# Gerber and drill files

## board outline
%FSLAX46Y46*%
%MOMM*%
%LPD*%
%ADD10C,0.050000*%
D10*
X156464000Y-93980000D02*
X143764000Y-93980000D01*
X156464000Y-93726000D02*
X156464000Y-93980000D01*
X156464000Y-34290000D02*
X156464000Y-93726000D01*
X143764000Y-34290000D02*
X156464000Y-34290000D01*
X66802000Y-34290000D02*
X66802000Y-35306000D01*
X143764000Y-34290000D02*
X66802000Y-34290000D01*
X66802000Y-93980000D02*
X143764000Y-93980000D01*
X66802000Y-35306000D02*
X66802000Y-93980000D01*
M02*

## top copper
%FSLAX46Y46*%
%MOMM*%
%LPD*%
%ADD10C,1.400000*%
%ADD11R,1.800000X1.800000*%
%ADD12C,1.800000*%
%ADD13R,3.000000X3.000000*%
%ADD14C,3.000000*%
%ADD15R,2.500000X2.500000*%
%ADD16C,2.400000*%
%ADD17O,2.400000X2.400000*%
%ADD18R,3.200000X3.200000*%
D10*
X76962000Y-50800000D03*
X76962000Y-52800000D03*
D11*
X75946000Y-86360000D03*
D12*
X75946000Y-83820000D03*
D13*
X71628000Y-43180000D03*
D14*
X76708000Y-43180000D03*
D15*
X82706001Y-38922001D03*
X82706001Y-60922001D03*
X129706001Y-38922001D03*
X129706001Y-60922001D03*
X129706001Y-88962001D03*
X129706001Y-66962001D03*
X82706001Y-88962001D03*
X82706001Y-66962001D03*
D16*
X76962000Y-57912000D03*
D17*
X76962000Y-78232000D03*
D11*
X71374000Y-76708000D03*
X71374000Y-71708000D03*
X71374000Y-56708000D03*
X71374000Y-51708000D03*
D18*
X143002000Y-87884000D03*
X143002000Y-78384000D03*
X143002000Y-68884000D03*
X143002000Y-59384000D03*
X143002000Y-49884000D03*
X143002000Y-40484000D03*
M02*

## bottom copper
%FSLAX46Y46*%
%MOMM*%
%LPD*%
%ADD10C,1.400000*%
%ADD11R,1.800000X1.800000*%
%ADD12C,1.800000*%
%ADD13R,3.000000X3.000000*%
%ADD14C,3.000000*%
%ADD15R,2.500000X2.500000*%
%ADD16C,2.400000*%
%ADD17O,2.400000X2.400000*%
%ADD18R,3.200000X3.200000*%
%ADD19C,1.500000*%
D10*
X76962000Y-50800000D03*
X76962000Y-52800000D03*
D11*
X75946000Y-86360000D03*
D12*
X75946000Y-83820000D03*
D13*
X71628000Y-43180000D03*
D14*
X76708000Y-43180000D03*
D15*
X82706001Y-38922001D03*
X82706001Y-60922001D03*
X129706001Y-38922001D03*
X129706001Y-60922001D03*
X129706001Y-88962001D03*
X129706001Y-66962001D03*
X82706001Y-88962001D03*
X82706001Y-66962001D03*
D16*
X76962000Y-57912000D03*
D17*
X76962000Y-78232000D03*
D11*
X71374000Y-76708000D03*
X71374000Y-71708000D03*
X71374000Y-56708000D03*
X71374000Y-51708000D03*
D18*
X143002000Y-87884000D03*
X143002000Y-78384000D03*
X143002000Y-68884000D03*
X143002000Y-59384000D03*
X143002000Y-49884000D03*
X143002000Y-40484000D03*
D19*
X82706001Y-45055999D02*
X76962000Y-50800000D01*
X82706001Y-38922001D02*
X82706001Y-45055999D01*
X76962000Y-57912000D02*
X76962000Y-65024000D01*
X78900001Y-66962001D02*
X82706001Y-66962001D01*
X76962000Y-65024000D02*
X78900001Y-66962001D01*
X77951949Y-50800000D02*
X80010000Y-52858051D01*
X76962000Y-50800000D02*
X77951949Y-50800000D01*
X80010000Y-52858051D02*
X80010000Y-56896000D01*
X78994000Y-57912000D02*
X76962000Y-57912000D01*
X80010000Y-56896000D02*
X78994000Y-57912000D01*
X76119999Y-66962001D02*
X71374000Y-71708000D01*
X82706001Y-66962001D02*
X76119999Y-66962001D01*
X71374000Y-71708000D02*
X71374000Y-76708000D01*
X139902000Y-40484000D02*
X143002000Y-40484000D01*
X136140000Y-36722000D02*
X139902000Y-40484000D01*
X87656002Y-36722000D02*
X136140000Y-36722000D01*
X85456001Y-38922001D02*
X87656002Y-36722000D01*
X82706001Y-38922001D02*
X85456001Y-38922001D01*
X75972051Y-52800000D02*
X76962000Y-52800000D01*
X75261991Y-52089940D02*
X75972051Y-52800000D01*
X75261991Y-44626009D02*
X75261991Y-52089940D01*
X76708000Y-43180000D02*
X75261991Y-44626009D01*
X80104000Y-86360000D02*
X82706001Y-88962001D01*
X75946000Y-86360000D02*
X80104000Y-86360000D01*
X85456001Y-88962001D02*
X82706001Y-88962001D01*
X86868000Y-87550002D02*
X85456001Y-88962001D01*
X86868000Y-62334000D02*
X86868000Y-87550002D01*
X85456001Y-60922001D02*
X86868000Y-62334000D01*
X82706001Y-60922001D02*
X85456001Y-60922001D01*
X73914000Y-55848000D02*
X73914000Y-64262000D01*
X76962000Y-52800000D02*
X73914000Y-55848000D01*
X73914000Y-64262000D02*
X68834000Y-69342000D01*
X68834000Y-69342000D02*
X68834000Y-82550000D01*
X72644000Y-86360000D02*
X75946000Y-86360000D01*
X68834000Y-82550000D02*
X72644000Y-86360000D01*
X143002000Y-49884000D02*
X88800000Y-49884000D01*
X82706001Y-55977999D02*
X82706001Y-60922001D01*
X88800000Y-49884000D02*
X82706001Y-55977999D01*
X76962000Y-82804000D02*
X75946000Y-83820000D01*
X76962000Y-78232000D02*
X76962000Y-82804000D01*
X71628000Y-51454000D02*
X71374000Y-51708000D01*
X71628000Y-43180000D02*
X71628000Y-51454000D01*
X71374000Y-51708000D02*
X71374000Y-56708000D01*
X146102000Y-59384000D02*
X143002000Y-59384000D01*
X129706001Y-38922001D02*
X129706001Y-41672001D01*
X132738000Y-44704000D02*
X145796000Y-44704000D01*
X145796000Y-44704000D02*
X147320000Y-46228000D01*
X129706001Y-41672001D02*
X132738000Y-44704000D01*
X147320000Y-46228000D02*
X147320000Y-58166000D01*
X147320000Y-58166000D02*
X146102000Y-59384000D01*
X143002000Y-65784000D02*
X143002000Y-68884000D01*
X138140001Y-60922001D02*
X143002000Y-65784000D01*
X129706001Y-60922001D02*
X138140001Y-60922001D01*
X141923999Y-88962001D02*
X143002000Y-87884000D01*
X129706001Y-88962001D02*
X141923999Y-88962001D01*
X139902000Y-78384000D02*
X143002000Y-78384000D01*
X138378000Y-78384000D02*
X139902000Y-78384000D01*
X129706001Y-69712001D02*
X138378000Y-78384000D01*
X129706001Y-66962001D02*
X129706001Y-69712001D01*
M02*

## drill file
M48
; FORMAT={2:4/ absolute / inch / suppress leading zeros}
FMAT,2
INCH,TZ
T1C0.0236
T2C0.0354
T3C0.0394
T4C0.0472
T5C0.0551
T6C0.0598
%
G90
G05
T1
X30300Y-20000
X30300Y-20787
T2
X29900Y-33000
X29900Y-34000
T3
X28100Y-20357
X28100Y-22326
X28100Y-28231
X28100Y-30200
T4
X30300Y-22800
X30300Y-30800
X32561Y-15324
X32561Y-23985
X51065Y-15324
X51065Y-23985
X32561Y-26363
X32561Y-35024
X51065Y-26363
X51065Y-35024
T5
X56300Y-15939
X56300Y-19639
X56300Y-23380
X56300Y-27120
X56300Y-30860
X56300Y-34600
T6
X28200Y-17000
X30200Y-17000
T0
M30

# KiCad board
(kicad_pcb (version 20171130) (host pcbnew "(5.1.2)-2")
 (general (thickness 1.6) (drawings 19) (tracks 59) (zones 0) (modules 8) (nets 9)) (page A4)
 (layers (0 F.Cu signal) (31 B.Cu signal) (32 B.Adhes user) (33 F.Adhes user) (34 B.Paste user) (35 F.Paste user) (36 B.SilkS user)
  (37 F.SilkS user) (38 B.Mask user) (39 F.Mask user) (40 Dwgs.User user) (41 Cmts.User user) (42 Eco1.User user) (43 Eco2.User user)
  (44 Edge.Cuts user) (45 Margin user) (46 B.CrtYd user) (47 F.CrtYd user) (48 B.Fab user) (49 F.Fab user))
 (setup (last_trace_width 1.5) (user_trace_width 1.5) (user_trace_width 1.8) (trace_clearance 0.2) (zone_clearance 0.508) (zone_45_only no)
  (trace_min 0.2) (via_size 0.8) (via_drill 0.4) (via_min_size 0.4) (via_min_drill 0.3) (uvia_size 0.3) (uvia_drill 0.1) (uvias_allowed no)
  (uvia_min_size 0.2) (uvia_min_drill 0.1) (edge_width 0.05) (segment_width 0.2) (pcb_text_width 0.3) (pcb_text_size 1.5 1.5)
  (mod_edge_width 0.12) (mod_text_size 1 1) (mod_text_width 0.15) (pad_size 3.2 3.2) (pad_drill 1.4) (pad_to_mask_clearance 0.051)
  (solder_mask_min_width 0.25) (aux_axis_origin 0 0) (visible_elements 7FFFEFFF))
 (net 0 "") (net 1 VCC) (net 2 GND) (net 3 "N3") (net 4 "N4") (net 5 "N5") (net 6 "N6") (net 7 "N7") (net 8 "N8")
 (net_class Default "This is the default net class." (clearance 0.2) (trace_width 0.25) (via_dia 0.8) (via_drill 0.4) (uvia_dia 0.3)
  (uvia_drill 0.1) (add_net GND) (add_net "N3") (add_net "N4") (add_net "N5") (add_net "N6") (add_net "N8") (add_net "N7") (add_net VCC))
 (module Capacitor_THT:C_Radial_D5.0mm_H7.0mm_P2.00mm (layer F.Cu) (at 76.962 50.8 270)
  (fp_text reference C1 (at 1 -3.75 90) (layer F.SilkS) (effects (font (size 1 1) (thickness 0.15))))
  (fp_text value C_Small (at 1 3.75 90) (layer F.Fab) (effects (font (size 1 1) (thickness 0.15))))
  (pad 1 thru_hole circle (at 0 0 270) (size 1.4 1.4) (drill 0.6) (layers *.Cu *.Mask) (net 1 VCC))
  (pad 2 thru_hole circle (at 2 0 270) (size 1.4 1.4) (drill 0.6) (layers *.Cu *.Mask) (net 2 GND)))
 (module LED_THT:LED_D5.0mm (layer F.Cu) (at 75.946 86.36 90)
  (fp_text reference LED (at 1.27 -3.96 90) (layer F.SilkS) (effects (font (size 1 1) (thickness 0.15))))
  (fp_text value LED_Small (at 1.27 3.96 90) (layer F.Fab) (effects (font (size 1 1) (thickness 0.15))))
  (pad 1 thru_hole rect (at 0 0 90) (size 1.8 1.8) (drill 0.9) (layers *.Cu *.Mask) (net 2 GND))
  (pad 2 thru_hole circle (at 2.54 0 90) (size 1.8 1.8) (drill 0.9) (layers *.Cu *.Mask) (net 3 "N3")))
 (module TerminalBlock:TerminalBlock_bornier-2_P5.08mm (layer F.Cu) (at 71.628 43.18)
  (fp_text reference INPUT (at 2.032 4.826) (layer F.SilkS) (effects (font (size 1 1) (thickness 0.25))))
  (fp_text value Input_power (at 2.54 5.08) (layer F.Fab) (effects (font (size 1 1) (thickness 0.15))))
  (pad 1 thru_hole rect (at 0 0) (size 3 3) (drill 1.52) (layers *.Cu *.Mask) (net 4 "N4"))
  (pad 2 thru_hole circle (at 5.08 0) (size 3 3) (drill 1.52) (layers *.Cu *.Mask) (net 2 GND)))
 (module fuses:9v (layer F.Cu) (at 82.706001 38.922001)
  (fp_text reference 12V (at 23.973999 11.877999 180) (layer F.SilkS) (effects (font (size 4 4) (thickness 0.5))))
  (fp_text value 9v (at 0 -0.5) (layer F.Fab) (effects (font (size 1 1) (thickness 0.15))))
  (pad 1 thru_hole rect (at 0 0) (size 2.5 2.5) (drill 1.2) (layers *.Cu *.Mask) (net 1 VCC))
  (pad 3 thru_hole rect (at 0 22) (size 2.5 2.5) (drill 1.2) (layers *.Cu *.Mask) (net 2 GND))
  (pad 2 thru_hole rect (at 47 0) (size 2.5 2.5) (drill 1.2) (layers *.Cu *.Mask) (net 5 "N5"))
  (pad 4 thru_hole rect (at 47 22) (size 2.5 2.5) (drill 1.2) (layers *.Cu *.Mask) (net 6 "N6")))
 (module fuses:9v (layer F.Cu) (at 82.706001 66.962001)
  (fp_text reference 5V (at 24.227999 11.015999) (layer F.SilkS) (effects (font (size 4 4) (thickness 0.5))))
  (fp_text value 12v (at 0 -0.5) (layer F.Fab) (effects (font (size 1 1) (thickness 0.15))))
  (pad 4 thru_hole rect (at 47 22) (size 2.5 2.5) (drill 1.2) (layers *.Cu *.Mask) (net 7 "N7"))
  (pad 2 thru_hole rect (at 47 0) (size 2.5 2.5) (drill 1.2) (layers *.Cu *.Mask) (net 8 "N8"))
  (pad 3 thru_hole rect (at 0 22) (size 2.5 2.5) (drill 1.2) (layers *.Cu *.Mask) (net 2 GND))
  (pad 1 thru_hole rect (at 0 0) (size 2.5 2.5) (drill 1.2) (layers *.Cu *.Mask) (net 1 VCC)))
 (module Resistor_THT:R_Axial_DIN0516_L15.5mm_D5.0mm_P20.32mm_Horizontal (layer F.Cu) (at 76.962 57.912 270)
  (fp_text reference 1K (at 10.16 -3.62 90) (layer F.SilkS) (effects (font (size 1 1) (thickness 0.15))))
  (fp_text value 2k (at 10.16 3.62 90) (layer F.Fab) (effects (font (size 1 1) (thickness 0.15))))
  (pad 1 thru_hole circle (at 0 0 270) (size 2.4 2.4) (drill 1.2) (layers *.Cu *.Mask) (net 1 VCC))
  (pad 2 thru_hole oval (at 20.32 0 270) (size 2.4 2.4) (drill 1.2) (layers *.Cu *.Mask) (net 3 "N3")))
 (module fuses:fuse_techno (layer F.Cu) (at 71.374 76.708 90)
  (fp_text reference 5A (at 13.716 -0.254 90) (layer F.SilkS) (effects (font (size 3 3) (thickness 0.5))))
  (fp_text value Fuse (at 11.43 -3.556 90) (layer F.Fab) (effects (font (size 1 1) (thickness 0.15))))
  (pad 1 thru_hole rect (at 0 0 90) (size 1.8 1.8) (drill 1) (layers *.Cu *.Mask) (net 1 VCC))
  (pad 1 thru_hole rect (at 5 0 90) (size 1.8 1.8) (drill 1) (layers *.Cu *.Mask) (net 1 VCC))
  (pad 2 thru_hole rect (at 20 0 90) (size 1.8 1.8) (drill 1) (layers *.Cu *.Mask) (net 4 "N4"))
  (pad 2 thru_hole rect (at 25 0 90) (size 1.8 1.8) (drill 1) (layers *.Cu *.Mask) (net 4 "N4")))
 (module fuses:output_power (layer F.Cu) (at 143.002 87.884 180)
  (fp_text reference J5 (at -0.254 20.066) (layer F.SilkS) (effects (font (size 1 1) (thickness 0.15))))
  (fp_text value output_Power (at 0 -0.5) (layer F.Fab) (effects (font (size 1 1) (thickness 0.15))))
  (pad 1 thru_hole rect (at 0 0 180) (size 3.2 3.2) (drill 1.4) (layers *.Cu *.Mask) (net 7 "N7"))
  (pad 2 thru_hole rect (at 0 9.5 180) (size 3.2 3.2) (drill 1.4) (layers *.Cu *.Mask) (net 8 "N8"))
  (pad 3 thru_hole rect (at 0 19 180) (size 3.2 3.2) (drill 1.4) (layers *.Cu *.Mask) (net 6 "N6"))
  (pad 4 thru_hole rect (at 0 28.5 180) (size 3.2 3.2) (drill 1.4) (layers *.Cu *.Mask) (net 5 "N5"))
  (pad 5 thru_hole rect (at 0 38 180) (size 3.2 3.2) (drill 1.4) (layers *.Cu *.Mask) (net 2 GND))
  (pad 6 thru_hole rect (at 0 47.4 180) (size 3.2 3.2) (drill 1.4) (layers *.Cu *.Mask) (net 1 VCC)))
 (gr_line (start 156.464 93.98) (end 143.764 93.98) (layer Edge.Cuts) (width 0.05))
 (gr_line (start 156.464 93.726) (end 156.464 93.98) (layer Edge.Cuts) (width 0.05))
 (gr_line (start 156.464 34.29) (end 156.464 93.726) (layer Edge.Cuts) (width 0.05))
 (gr_line (start 143.764 34.29) (end 156.464 34.29) (layer Edge.Cuts) (width 0.05))
 (gr_line (start 66.802 34.29) (end 66.802 35.306) (layer Edge.Cuts) (width 0.05))
 (gr_line (start 143.764 34.29) (end 66.802 34.29) (layer Edge.Cuts) (width 0.05))
 (gr_line (start 66.802 93.98) (end 143.764 93.98) (layer Edge.Cuts) (width 0.05))
 (gr_line (start 66.802 35.306) (end 66.802 93.98) (layer Edge.Cuts) (width 0.05))
 (segment (start 82.706001 45.055999) (end 76.962 50.8) (width 1.5) (layer B.Cu) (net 1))
 (segment (start 82.706001 38.922001) (end 82.706001 45.055999) (width 1.5) (layer B.Cu) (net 1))
 (segment (start 76.962 57.912) (end 76.962 65.024) (width 1.5) (layer B.Cu) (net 1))
 (segment (start 78.900001 66.962001) (end 82.706001 66.962001) (width 1.5) (layer B.Cu) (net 1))
 (segment (start 76.962 65.024) (end 78.900001 66.962001) (width 1.5) (layer B.Cu) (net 1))
 (segment (start 77.951949 50.8) (end 80.01 52.858051) (width 1.5) (layer B.Cu) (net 1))
 (segment (start 76.962 50.8) (end 77.951949 50.8) (width 1.5) (layer B.Cu) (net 1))
 (segment (start 80.01 52.858051) (end 80.01 56.896) (width 1.5) (layer B.Cu) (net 1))
 (segment (start 78.994 57.912) (end 76.962 57.912) (width 1.5) (layer B.Cu) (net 1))
 (segment (start 80.01 56.896) (end 78.994 57.912) (width 1.5) (layer B.Cu) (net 1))
 (segment (start 76.119999 66.962001) (end 71.374 71.708) (width 1.5) (layer B.Cu) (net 1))
 (segment (start 82.706001 66.962001) (end 76.119999 66.962001) (width 1.5) (layer B.Cu) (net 1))
 (segment (start 71.374 71.708) (end 71.374 76.708) (width 1.5) (layer B.Cu) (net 1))
 (segment (start 139.902 40.484) (end 143.002 40.484) (width 1.5) (layer B.Cu) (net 1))
 (segment (start 136.14 36.722) (end 139.902 40.484) (width 1.5) (layer B.Cu) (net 1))
 (segment (start 87.656002 36.722) (end 136.14 36.722) (width 1.5) (layer B.Cu) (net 1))
 (segment (start 85.456001 38.922001) (end 87.656002 36.722) (width 1.5) (layer B.Cu) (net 1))
 (segment (start 82.706001 38.922001) (end 85.456001 38.922001) (width 1.5) (layer B.Cu) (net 1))
 (segment (start 75.972051 52.8) (end 76.962 52.8) (width 1.5) (layer B.Cu) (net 2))
 (segment (start 75.261991 52.08994) (end 75.972051 52.8) (width 1.5) (layer B.Cu) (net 2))
 (segment (start 75.261991 44.626009) (end 75.261991 52.08994) (width 1.5) (layer B.Cu) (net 2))
 (segment (start 76.708 43.18) (end 75.261991 44.626009) (width 1.5) (layer B.Cu) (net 2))
 (segment (start 80.104 86.36) (end 82.706001 88.962001) (width 1.5) (layer B.Cu) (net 2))
 (segment (start 75.946 86.36) (end 80.104 86.36) (width 1.5) (layer B.Cu) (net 2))
 (segment (start 85.456001 88.962001) (end 82.706001 88.962001) (width 1.5) (layer B.Cu) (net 2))
 (segment (start 86.868 87.550002) (end 85.456001 88.962001) (width 1.5) (layer B.Cu) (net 2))
 (segment (start 86.868 62.334) (end 86.868 87.550002) (width 1.5) (layer B.Cu) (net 2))
 (segment (start 85.456001 60.922001) (end 86.868 62.334) (width 1.5) (layer B.Cu) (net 2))
 (segment (start 82.706001 60.922001) (end 85.456001 60.922001) (width 1.5) (layer B.Cu) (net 2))
 (segment (start 73.914 55.848) (end 73.914 64.262) (width 1.5) (layer B.Cu) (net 2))
 (segment (start 76.962 52.8) (end 73.914 55.848) (width 1.5) (layer B.Cu) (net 2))
 (segment (start 73.914 64.262) (end 68.834 69.342) (width 1.5) (layer B.Cu) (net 2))
 (segment (start 68.834 69.342) (end 68.834 82.55) (width 1.5) (layer B.Cu) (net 2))
 (segment (start 72.644 86.36) (end 75.946 86.36) (width 1.5) (layer B.Cu) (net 2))
 (segment (start 68.834 82.55) (end 72.644 86.36) (width 1.5) (layer B.Cu) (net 2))
 (segment (start 143.002 49.884) (end 88.8 49.884) (width 1.5) (layer B.Cu) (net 2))
 (segment (start 82.706001 55.977999) (end 82.706001 60.922001) (width 1.5) (layer B.Cu) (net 2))
 (segment (start 88.8 49.884) (end 82.706001 55.977999) (width 1.5) (layer B.Cu) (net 2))
 (segment (start 76.962 82.804) (end 75.946 83.82) (width 1.5) (layer B.Cu) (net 3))
 (segment (start 76.962 78.232) (end 76.962 82.804) (width 1.5) (layer B.Cu) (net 3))
 (segment (start 71.628 51.454) (end 71.374 51.708) (width 1.5) (layer B.Cu) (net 4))
 (segment (start 71.628 43.18) (end 71.628 51.454) (width 1.5) (layer B.Cu) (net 4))
 (segment (start 71.374 51.708) (end 71.374 56.708) (width 1.5) (layer B.Cu) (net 4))
 (segment (start 146.102 59.384) (end 143.002 59.384) (width 1.5) (layer B.Cu) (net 5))
 (segment (start 129.706001 38.922001) (end 129.706001 41.672001) (width 1.5) (layer B.Cu) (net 5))
 (segment (start 132.738 44.704) (end 145.796 44.704) (width 1.5) (layer B.Cu) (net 5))
 (segment (start 145.796 44.704) (end 147.32 46.228) (width 1.5) (layer B.Cu) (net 5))
 (segment (start 129.706001 41.672001) (end 132.738 44.704) (width 1.5) (layer B.Cu) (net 5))
 (segment (start 147.32 46.228) (end 147.32 58.166) (width 1.5) (layer B.Cu) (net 5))
 (segment (start 147.32 58.166) (end 146.102 59.384) (width 1.5) (layer B.Cu) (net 5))
 (segment (start 143.002 65.784) (end 143.002 68.884) (width 1.5) (layer B.Cu) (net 6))
 (segment (start 138.140001 60.922001) (end 143.002 65.784) (width 1.5) (layer B.Cu) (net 6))
 (segment (start 129.706001 60.922001) (end 138.140001 60.922001) (width 1.5) (layer B.Cu) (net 6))
 (segment (start 141.923999 88.962001) (end 143.002 87.884) (width 1.5) (layer B.Cu) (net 7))
 (segment (start 129.706001 88.962001) (end 141.923999 88.962001) (width 1.5) (layer B.Cu) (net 7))
 (segment (start 139.902 78.384) (end 143.002 78.384) (width 1.5) (layer B.Cu) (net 8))
 (segment (start 138.378 78.384) (end 139.902 78.384) (width 1.5) (layer B.Cu) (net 8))
 (segment (start 129.706001 69.712001) (end 138.378 78.384) (width 1.5) (layer B.Cu) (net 8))
 (segment (start 129.706001 66.962001) (end 129.706001 69.712001) (width 1.5) (layer B.Cu) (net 8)))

